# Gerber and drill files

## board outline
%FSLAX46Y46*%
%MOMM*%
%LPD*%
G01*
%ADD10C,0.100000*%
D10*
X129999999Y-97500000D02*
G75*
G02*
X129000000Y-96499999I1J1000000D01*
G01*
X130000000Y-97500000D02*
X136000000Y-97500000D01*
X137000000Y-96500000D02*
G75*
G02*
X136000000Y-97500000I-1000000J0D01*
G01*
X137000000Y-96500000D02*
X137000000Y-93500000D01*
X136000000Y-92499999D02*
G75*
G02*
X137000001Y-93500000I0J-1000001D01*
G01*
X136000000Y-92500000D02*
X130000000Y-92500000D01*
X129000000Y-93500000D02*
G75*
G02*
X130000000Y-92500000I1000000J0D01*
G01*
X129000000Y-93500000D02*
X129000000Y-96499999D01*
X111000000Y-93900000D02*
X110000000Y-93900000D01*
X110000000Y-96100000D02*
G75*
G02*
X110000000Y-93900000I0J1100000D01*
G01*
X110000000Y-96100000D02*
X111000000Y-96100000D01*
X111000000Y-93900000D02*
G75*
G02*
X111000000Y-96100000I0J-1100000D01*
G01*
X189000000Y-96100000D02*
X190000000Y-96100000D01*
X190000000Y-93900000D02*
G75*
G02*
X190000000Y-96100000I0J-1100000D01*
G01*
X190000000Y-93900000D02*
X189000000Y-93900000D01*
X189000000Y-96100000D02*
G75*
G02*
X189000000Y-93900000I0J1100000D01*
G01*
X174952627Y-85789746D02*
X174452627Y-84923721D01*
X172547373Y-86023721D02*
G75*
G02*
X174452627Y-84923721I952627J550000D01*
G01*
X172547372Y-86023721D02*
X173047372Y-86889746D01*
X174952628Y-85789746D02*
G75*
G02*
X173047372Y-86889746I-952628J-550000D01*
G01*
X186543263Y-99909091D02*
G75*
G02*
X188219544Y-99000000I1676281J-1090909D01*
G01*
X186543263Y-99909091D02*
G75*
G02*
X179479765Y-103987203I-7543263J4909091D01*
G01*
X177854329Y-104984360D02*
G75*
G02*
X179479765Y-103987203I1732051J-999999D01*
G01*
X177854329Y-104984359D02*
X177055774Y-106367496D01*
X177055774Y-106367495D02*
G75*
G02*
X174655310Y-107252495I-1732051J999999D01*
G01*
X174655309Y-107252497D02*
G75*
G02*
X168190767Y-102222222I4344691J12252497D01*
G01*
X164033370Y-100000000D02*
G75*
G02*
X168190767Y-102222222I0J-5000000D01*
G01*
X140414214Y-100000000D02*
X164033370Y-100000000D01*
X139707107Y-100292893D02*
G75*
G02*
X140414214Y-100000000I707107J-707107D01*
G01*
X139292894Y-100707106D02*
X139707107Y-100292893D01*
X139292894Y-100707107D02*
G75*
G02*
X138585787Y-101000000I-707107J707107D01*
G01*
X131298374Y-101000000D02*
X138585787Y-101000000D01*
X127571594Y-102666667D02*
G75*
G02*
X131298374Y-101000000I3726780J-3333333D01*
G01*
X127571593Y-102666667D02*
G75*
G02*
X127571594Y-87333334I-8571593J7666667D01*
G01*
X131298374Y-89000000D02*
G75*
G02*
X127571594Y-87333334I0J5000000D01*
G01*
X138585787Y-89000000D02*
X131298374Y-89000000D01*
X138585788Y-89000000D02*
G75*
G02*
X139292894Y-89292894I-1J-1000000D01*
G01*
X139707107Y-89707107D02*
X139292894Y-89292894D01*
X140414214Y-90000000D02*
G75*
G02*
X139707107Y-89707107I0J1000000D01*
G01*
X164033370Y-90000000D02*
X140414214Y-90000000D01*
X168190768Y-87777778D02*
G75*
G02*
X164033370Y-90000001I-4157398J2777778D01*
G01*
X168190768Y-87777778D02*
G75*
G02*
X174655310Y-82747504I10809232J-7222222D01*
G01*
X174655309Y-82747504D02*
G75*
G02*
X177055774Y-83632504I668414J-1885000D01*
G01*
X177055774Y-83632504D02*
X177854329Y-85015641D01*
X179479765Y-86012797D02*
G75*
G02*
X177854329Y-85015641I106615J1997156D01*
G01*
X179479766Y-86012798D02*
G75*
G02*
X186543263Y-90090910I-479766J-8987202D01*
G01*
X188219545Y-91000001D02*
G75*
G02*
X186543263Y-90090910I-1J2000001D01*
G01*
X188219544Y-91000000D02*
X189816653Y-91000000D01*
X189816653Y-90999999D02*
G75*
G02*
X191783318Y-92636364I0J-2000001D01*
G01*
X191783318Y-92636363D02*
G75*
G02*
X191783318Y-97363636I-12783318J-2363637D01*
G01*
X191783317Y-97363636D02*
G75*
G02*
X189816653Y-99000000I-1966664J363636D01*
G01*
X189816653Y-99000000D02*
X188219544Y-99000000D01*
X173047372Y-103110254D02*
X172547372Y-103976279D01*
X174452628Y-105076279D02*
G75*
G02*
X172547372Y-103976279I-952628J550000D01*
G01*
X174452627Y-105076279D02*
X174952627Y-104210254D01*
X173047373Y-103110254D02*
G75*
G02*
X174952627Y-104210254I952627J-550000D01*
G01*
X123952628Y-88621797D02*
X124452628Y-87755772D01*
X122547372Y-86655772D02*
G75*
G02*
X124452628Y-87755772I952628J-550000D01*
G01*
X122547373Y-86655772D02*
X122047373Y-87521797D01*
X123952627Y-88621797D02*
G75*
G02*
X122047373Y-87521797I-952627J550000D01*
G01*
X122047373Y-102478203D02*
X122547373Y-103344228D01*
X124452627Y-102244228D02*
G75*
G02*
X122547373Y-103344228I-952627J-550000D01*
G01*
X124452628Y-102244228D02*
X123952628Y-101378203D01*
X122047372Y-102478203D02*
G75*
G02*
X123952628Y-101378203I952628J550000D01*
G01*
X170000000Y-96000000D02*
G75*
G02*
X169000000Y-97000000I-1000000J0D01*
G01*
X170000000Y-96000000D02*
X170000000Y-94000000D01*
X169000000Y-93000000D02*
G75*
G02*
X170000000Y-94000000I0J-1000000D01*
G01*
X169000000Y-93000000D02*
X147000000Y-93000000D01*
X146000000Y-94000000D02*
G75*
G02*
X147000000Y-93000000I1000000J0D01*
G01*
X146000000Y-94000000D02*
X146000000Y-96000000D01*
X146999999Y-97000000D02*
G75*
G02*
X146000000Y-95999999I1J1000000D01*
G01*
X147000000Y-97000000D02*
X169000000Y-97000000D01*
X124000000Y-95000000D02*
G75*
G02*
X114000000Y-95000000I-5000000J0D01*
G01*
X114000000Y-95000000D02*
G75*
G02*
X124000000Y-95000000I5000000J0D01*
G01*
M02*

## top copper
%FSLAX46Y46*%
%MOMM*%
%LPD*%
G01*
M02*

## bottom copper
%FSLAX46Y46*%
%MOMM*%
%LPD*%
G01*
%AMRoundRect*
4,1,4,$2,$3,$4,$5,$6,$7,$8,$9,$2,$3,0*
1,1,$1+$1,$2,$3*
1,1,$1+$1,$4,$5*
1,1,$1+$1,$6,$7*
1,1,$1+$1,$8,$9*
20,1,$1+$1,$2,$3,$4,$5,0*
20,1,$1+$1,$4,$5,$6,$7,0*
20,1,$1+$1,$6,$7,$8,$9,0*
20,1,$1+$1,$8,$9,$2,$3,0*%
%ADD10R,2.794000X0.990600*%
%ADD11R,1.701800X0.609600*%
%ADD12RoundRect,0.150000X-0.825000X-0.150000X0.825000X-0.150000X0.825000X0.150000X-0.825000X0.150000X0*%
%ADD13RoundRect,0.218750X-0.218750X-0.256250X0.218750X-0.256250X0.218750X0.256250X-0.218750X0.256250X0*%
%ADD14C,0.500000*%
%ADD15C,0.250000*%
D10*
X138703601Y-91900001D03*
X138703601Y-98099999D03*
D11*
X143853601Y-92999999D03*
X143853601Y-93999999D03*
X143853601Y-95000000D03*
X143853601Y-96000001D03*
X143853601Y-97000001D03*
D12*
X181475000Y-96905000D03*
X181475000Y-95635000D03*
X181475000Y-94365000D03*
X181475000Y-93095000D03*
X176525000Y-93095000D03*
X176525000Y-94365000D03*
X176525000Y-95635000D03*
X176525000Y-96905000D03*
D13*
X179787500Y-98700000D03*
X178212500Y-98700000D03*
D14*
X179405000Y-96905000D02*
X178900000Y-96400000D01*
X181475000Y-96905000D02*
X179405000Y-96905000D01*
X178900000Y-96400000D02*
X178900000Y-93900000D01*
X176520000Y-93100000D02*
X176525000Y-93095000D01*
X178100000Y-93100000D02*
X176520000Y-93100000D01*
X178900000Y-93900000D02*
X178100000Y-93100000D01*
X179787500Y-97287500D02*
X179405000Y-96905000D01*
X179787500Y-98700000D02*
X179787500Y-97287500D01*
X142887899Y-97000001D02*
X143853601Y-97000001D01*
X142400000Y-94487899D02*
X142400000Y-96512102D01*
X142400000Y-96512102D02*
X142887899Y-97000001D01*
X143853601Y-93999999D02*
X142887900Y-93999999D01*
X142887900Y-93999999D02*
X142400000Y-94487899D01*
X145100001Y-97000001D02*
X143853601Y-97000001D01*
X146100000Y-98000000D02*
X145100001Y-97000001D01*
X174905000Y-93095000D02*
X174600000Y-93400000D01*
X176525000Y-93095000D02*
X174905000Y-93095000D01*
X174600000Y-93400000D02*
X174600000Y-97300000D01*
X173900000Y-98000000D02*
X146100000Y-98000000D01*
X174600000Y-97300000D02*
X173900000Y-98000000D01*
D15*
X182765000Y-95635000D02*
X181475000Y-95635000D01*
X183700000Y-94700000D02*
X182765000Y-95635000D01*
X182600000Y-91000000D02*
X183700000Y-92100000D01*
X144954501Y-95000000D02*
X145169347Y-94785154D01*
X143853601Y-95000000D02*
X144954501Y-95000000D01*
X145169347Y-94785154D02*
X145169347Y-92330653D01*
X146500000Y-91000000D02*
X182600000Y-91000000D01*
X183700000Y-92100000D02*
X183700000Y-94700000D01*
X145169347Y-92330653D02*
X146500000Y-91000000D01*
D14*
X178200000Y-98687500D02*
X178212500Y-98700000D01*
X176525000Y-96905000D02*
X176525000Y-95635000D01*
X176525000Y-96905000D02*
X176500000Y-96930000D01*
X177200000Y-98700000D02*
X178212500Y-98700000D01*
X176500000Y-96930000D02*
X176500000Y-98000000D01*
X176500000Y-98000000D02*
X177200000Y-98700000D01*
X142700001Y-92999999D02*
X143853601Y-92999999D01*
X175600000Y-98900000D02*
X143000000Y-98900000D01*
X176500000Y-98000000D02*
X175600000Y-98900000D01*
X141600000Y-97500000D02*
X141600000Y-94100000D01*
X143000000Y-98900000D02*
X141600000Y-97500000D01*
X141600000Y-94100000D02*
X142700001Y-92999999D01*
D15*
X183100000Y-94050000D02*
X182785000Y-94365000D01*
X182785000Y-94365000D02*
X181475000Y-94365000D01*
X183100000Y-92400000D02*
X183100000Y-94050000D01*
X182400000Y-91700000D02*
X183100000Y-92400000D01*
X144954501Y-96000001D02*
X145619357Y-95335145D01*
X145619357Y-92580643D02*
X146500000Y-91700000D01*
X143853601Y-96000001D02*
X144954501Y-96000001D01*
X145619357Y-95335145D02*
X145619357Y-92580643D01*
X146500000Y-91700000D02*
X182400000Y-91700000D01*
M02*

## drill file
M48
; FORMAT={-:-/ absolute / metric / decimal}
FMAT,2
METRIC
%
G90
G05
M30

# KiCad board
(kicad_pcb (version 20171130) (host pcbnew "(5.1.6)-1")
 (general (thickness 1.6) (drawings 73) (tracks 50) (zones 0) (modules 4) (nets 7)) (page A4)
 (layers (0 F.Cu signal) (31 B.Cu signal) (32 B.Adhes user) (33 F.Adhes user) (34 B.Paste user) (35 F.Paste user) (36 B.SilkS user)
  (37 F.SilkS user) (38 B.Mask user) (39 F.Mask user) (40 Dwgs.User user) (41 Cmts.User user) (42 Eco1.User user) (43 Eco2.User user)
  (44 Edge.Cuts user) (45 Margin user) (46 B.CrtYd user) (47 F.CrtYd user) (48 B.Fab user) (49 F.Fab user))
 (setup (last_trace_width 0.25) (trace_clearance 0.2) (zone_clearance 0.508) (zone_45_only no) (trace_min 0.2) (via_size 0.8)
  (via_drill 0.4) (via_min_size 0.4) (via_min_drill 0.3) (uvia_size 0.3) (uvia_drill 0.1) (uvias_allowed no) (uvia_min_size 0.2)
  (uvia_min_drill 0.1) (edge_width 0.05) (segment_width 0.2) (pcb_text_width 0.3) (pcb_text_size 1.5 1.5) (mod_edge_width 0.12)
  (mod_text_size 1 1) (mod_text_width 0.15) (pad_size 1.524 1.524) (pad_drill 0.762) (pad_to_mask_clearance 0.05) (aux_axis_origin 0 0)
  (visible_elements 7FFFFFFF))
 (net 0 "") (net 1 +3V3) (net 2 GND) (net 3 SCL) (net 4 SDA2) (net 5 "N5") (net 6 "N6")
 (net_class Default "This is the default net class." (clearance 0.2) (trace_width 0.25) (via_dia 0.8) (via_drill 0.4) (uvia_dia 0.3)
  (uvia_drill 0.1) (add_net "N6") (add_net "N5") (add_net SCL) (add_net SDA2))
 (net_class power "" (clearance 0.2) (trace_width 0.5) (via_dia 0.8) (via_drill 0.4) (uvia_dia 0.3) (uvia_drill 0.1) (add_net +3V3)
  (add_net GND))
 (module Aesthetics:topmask (layer F.Cu) (at 148.8 96.7)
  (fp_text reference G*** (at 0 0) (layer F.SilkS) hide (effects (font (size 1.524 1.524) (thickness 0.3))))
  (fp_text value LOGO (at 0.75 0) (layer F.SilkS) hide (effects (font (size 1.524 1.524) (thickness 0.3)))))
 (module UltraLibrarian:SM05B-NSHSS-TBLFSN (layer B.Cu) (at 141 95 90)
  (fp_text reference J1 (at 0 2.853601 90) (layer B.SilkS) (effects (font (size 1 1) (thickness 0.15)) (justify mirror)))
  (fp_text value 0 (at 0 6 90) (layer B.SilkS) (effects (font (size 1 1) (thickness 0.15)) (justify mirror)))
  (pad 7 smd rect (at 3.099999 -2.296399 90) (size 0.9906 2.794) (layers B.Cu B.Paste B.Mask))
  (pad 6 smd rect (at -3.099999 -2.296399 90) (size 0.9906 2.794) (layers B.Cu B.Paste B.Mask))
  (pad 5 smd rect (at 2.000001 2.853601 90) (size 0.6096 1.7018) (layers B.Cu B.Paste B.Mask) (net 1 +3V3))
  (pad 4 smd rect (at 1.000001 2.853601 90) (size 0.6096 1.7018) (layers B.Cu B.Paste B.Mask) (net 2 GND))
  (pad 3 smd rect (at 0 2.853601 90) (size 0.6096 1.7018) (layers B.Cu B.Paste B.Mask) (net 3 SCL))
  (pad 2 smd rect (at -1.000001 2.853601 90) (size 0.6096 1.7018) (layers B.Cu B.Paste B.Mask) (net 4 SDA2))
  (pad 1 smd rect (at -2.000001 2.853601 90) (size 0.6096 1.7018) (layers B.Cu B.Paste B.Mask) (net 2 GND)))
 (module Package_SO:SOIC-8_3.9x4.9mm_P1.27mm (layer B.Cu) (at 179 95)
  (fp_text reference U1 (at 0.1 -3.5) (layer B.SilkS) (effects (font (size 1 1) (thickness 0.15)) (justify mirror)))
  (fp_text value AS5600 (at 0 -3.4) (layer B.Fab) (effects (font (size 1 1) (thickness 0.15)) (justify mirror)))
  (pad 8 smd roundrect (at 2.475 1.905) (size 1.95 0.6) (layers B.Cu B.Paste B.Mask) (roundrect_rratio 0.25) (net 2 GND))
  (pad 7 smd roundrect (at 2.475 0.635) (size 1.95 0.6) (layers B.Cu B.Paste B.Mask) (roundrect_rratio 0.25) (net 3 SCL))
  (pad 6 smd roundrect (at 2.475 -0.635) (size 1.95 0.6) (layers B.Cu B.Paste B.Mask) (roundrect_rratio 0.25) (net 4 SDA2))
  (pad 5 smd roundrect (at 2.475 -1.905) (size 1.95 0.6) (layers B.Cu B.Paste B.Mask) (roundrect_rratio 0.25) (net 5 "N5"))
  (pad 4 smd roundrect (at -2.475 -1.905) (size 1.95 0.6) (layers B.Cu B.Paste B.Mask) (roundrect_rratio 0.25) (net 2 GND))
  (pad 3 smd roundrect (at -2.475 -0.635) (size 1.95 0.6) (layers B.Cu B.Paste B.Mask) (roundrect_rratio 0.25) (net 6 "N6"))
  (pad 2 smd roundrect (at -2.475 0.635) (size 1.95 0.6) (layers B.Cu B.Paste B.Mask) (roundrect_rratio 0.25) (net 1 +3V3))
  (pad 1 smd roundrect (at -2.475 1.905) (size 1.95 0.6) (layers B.Cu B.Paste B.Mask) (roundrect_rratio 0.25) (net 1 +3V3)))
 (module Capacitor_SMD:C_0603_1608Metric (layer B.Cu) (at 179 98.7)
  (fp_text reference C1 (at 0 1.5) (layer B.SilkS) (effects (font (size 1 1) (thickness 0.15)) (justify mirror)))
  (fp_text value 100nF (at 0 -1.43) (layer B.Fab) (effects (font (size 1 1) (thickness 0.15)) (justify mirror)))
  (pad 2 smd roundrect (at 0.7875 0) (size 0.875 0.95) (layers B.Cu B.Paste B.Mask) (roundrect_rratio 0.25) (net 2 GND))
  (pad 1 smd roundrect (at -0.7875 0) (size 0.875 0.95) (layers B.Cu B.Paste B.Mask) (roundrect_rratio 0.25) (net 1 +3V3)))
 (gr_arc (start 130 96.5) (end 129 96.499999) (angle -90) (layer Edge.Cuts) (width 0.1))
 (gr_line (start 130 97.5) (end 136 97.5) (layer Edge.Cuts) (width 0.1))
 (gr_arc (start 136 96.5) (end 136 97.5) (angle -90) (layer Edge.Cuts) (width 0.1))
 (gr_line (start 137 96.5) (end 137 93.5) (layer Edge.Cuts) (width 0.1))
 (gr_arc (start 136 93.5) (end 137.000001 93.5) (angle -90) (layer Edge.Cuts) (width 0.1))
 (gr_line (start 136 92.5) (end 130 92.5) (layer Edge.Cuts) (width 0.1))
 (gr_arc (start 130 93.5) (end 130 92.5) (angle -90) (layer Edge.Cuts) (width 0.1))
 (gr_line (start 129 93.5) (end 129 96.499999) (layer Edge.Cuts) (width 0.1))
 (gr_line (start 111 93.9) (end 110 93.9) (layer Edge.Cuts) (width 0.1))
 (gr_arc (start 110 95) (end 110 93.9) (angle -180) (layer Edge.Cuts) (width 0.1))
 (gr_line (start 110 96.1) (end 111 96.1) (layer Edge.Cuts) (width 0.1))
 (gr_arc (start 111 95) (end 111 96.1) (angle -180) (layer Edge.Cuts) (width 0.1))
 (gr_line (start 189 96.1) (end 190 96.1) (layer Edge.Cuts) (width 0.1))
 (gr_arc (start 190 95) (end 190 96.1) (angle -180) (layer Edge.Cuts) (width 0.1))
 (gr_line (start 190 93.9) (end 189 93.9) (layer Edge.Cuts) (width 0.1))
 (gr_arc (start 189 95) (end 189 93.9) (angle -180) (layer Edge.Cuts) (width 0.1))
 (gr_line (start 174.952627 85.789746) (end 174.452627 84.923721) (layer Edge.Cuts) (width 0.1))
 (gr_arc (start 173.5 85.473721) (end 174.452627 84.923721) (angle -180) (layer Edge.Cuts) (width 0.1))
 (gr_line (start 172.547372 86.023721) (end 173.047372 86.889746) (layer Edge.Cuts) (width 0.1))
 (gr_arc (start 174 86.339746) (end 173.047372 86.889746) (angle -180) (layer Edge.Cuts) (width 0.1))
 (gr_arc (start 188.219544 101) (end 188.219544 99) (angle -56.94426885) (layer Edge.Cuts) (width 0.1))
 (gr_arc (start 179 95) (end 179.479765 103.987203) (angle -53.8885377) (layer Edge.Cuts) (width 0.1))
 (gr_arc (start 179.58638 105.984359) (end 179.479765 103.987203) (angle -56.94426885) (layer Edge.Cuts) (width 0.1))
 (gr_line (start 177.854329 104.984359) (end 177.055774 106.367496) (layer Edge.Cuts) (width 0.1))
 (gr_arc (start 175.323723 105.367496) (end 174.65531 107.252496) (angle -79.5243183) (layer Edge.Cuts) (width 0.1))
 (gr_arc (start 179 95) (end 168.190767 102.222222) (angle -36.7266931) (layer Edge.Cuts) (width 0.1))
 (gr_arc (start 164.03337 105) (end 168.190767 102.222222) (angle -56.2510114) (layer Edge.Cuts) (width 0.1))
 (gr_line (start 140.414214 100) (end 164.03337 100) (layer Edge.Cuts) (width 0.1))
 (gr_arc (start 140.414214 101) (end 140.414214 99.999999) (angle -45) (layer Edge.Cuts) (width 0.1))
 (gr_line (start 139.292894 100.707106) (end 139.707107 100.292893) (layer Edge.Cuts) (width 0.1))
 (gr_arc (start 138.585787 100) (end 138.585787 101) (angle -45) (layer Edge.Cuts) (width 0.1))
 (gr_line (start 131.298374 101) (end 138.585787 101) (layer Edge.Cuts) (width 0.1))
 (gr_arc (start 131.298374 106) (end 131.298374 101) (angle -48.1896851) (layer Edge.Cuts) (width 0.1))
 (gr_arc (start 119 95) (end 127.571594 87.333334) (angle -276.3793702) (layer Edge.Cuts) (width 0.1))
 (gr_arc (start 131.298374 84) (end 127.571594 87.333334) (angle -48.1896851) (layer Edge.Cuts) (width 0.1))
 (gr_line (start 138.585787 89) (end 131.298374 89) (layer Edge.Cuts) (width 0.1))
 (gr_arc (start 138.585787 90) (end 139.292894 89.292894) (angle -45) (layer Edge.Cuts) (width 0.1))
 (gr_line (start 139.707107 89.707107) (end 139.292894 89.292894) (layer Edge.Cuts) (width 0.1))
 (gr_arc (start 140.414214 89) (end 139.707107 89.707107) (angle -45) (layer Edge.Cuts) (width 0.1))
 (gr_line (start 164.03337 90) (end 140.414214 90) (layer Edge.Cuts) (width 0.1))
 (gr_arc (start 164.03337 85) (end 164.03337 90.000001) (angle -56.2510114) (layer Edge.Cuts) (width 0.1))
 (gr_arc (start 179 95) (end 174.65531 82.747504) (angle -36.7266931) (layer Edge.Cuts) (width 0.1))
 (gr_arc (start 175.323723 84.632504) (end 177.055774 83.632504) (angle -79.5243183) (layer Edge.Cuts) (width 0.1))
 (gr_line (start 177.055774 83.632504) (end 177.854329 85.015641) (layer Edge.Cuts) (width 0.1))
 (gr_arc (start 179.58638 84.015641) (end 177.854329 85.015641) (angle -56.94426885) (layer Edge.Cuts) (width 0.1))
 (gr_arc (start 179 95) (end 186.543263 90.09091) (angle -53.8885377) (layer Edge.Cuts) (width 0.1))
 (gr_arc (start 188.219544 89) (end 186.543263 90.09091) (angle -56.94426885) (layer Edge.Cuts) (width 0.1))
 (gr_line (start 188.219544 91) (end 189.816653 91) (layer Edge.Cuts) (width 0.1))
 (gr_arc (start 189.816653 93) (end 191.783318 92.636364) (angle -79.5243183) (layer Edge.Cuts) (width 0.1))
 (gr_arc (start 179 95) (end 191.783318 97.363636) (angle -20.95136339) (layer Edge.Cuts) (width 0.1))
 (gr_arc (start 189.816653 97) (end 189.816653 99) (angle -79.5243183) (layer Edge.Cuts) (width 0.1))
 (gr_line (start 189.816653 99) (end 188.219544 99) (layer Edge.Cuts) (width 0.1))
 (gr_line (start 173.047372 103.110254) (end 172.547372 103.976279) (layer Edge.Cuts) (width 0.1))
 (gr_arc (start 173.5 104.526279) (end 172.547372 103.976279) (angle -180) (layer Edge.Cuts) (width 0.1))
 (gr_line (start 174.452627 105.076279) (end 174.952627 104.210254) (layer Edge.Cuts) (width 0.1))
 (gr_arc (start 174 103.660254) (end 174.952627 104.210254) (angle -180) (layer Edge.Cuts) (width 0.1))
 (gr_line (start 123.952628 88.621797) (end 124.452628 87.755772) (layer Edge.Cuts) (width 0.1))
 (gr_arc (start 123.5 87.205772) (end 124.452628 87.755772) (angle -180) (layer Edge.Cuts) (width 0.1))
 (gr_line (start 122.547373 86.655772) (end 122.047373 87.521797) (layer Edge.Cuts) (width 0.1))
 (gr_arc (start 123 88.071797) (end 122.047373 87.521797) (angle -180) (layer Edge.Cuts) (width 0.1))
 (gr_line (start 122.047373 102.478203) (end 122.547373 103.344228) (layer Edge.Cuts) (width 0.1))
 (gr_arc (start 123.5 102.794228) (end 122.547373 103.344228) (angle -180) (layer Edge.Cuts) (width 0.1))
 (gr_line (start 124.452628 102.244228) (end 123.952628 101.378203) (layer Edge.Cuts) (width 0.1))
 (gr_arc (start 123 101.928203) (end 123.952628 101.378203) (angle -180) (layer Edge.Cuts) (width 0.1))
 (gr_arc (start 169 96) (end 169 97) (angle -90) (layer Edge.Cuts) (width 0.1))
 (gr_line (start 170 96) (end 170 94) (layer Edge.Cuts) (width 0.1))
 (gr_arc (start 169 94) (end 170 94) (angle -90) (layer Edge.Cuts) (width 0.1))
 (gr_line (start 169 93) (end 147 93) (layer Edge.Cuts) (width 0.1))
 (gr_arc (start 147 94) (end 147 93) (angle -90) (layer Edge.Cuts) (width 0.1))
 (gr_line (start 146 94) (end 146 96) (layer Edge.Cuts) (width 0.1))
 (gr_arc (start 147 96) (end 146 95.999999) (angle -90) (layer Edge.Cuts) (width 0.1))
 (gr_line (start 147 97) (end 169 97) (layer Edge.Cuts) (width 0.1))
 (gr_circle (center 119 95) (end 124 95) (layer Edge.Cuts) (width 0.1))
 (segment (start 179.405 96.905) (end 178.9 96.4) (width 0.5) (layer B.Cu) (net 2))
 (segment (start 181.475 96.905) (end 179.405 96.905) (width 0.5) (layer B.Cu) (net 2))
 (segment (start 178.9 96.4) (end 178.9 93.9) (width 0.5) (layer B.Cu) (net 2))
 (segment (start 176.52 93.1) (end 176.525 93.095) (width 0.5) (layer B.Cu) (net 2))
 (segment (start 178.1 93.1) (end 176.52 93.1) (width 0.5) (layer B.Cu) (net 2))
 (segment (start 178.9 93.9) (end 178.1 93.1) (width 0.5) (layer B.Cu) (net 2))
 (segment (start 179.7875 97.2875) (end 179.405 96.905) (width 0.5) (layer B.Cu) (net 2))
 (segment (start 179.7875 98.7) (end 179.7875 97.2875) (width 0.5) (layer B.Cu) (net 2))
 (segment (start 142.887899 97.000001) (end 143.853601 97.000001) (width 0.5) (layer B.Cu) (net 2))
 (segment (start 142.4 94.487899) (end 142.4 96.512102) (width 0.5) (layer B.Cu) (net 2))
 (segment (start 142.4 96.512102) (end 142.887899 97.000001) (width 0.5) (layer B.Cu) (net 2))
 (segment (start 143.853601 93.999999) (end 142.8879 93.999999) (width 0.5) (layer B.Cu) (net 2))
 (segment (start 142.8879 93.999999) (end 142.4 94.487899) (width 0.5) (layer B.Cu) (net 2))
 (segment (start 145.100001 97.000001) (end 143.853601 97.000001) (width 0.5) (layer B.Cu) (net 2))
 (segment (start 146.1 98) (end 145.100001 97.000001) (width 0.5) (layer B.Cu) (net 2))
 (segment (start 174.905 93.095) (end 174.6 93.4) (width 0.5) (layer B.Cu) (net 2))
 (segment (start 176.525 93.095) (end 174.905 93.095) (width 0.5) (layer B.Cu) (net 2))
 (segment (start 174.6 93.4) (end 174.6 97.3) (width 0.5) (layer B.Cu) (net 2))
 (segment (start 173.9 98) (end 146.1 98) (width 0.5) (layer B.Cu) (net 2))
 (segment (start 174.6 97.3) (end 173.9 98) (width 0.5) (layer B.Cu) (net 2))
 (segment (start 182.765 95.635) (end 181.475 95.635) (width 0.25) (layer B.Cu) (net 3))
 (segment (start 183.7 94.7) (end 182.765 95.635) (width 0.25) (layer B.Cu) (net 3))
 (segment (start 182.6 91) (end 183.7 92.1) (width 0.25) (layer B.Cu) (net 3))
 (segment (start 144.954501 95) (end 145.169347 94.785154) (width 0.25) (layer B.Cu) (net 3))
 (segment (start 143.853601 95) (end 144.954501 95) (width 0.25) (layer B.Cu) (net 3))
 (segment (start 145.169347 94.785154) (end 145.169347 92.330653) (width 0.25) (layer B.Cu) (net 3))
 (segment (start 146.5 91) (end 182.6 91) (width 0.25) (layer B.Cu) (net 3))
 (segment (start 183.7 92.1) (end 183.7 94.7) (width 0.25) (layer B.Cu) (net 3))
 (segment (start 145.169347 92.330653) (end 146.5 91) (width 0.25) (layer B.Cu) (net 3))
 (segment (start 178.2 98.6875) (end 178.2125 98.7) (width 0.5) (layer B.Cu) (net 1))
 (segment (start 176.525 96.905) (end 176.525 95.635) (width 0.5) (layer B.Cu) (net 1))
 (segment (start 176.525 96.905) (end 176.5 96.93) (width 0.5) (layer B.Cu) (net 1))
 (segment (start 177.2 98.7) (end 178.2125 98.7) (width 0.5) (layer B.Cu) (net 1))
 (segment (start 176.5 96.93) (end 176.5 98) (width 0.5) (layer B.Cu) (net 1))
 (segment (start 176.5 98) (end 177.2 98.7) (width 0.5) (layer B.Cu) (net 1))
 (segment (start 142.700001 92.999999) (end 143.853601 92.999999) (width 0.5) (layer B.Cu) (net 1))
 (segment (start 175.6 98.9) (end 143 98.9) (width 0.5) (layer B.Cu) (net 1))
 (segment (start 176.5 98) (end 175.6 98.9) (width 0.5) (layer B.Cu) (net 1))
 (segment (start 141.6 97.5) (end 141.6 94.1) (width 0.5) (layer B.Cu) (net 1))
 (segment (start 143 98.9) (end 141.6 97.5) (width 0.5) (layer B.Cu) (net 1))
 (segment (start 141.6 94.1) (end 142.700001 92.999999) (width 0.5) (layer B.Cu) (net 1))
 (segment (start 183.1 94.05) (end 182.785 94.365) (width 0.25) (layer B.Cu) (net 4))
 (segment (start 182.785 94.365) (end 181.475 94.365) (width 0.25) (layer B.Cu) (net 4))
 (segment (start 183.1 92.4) (end 183.1 94.05) (width 0.25) (layer B.Cu) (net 4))
 (segment (start 182.4 91.7) (end 183.1 92.4) (width 0.25) (layer B.Cu) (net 4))
 (segment (start 144.954501 96.000001) (end 145.619357 95.335145) (width 0.25) (layer B.Cu) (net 4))
 (segment (start 145.619357 92.580643) (end 146.5 91.7) (width 0.25) (layer B.Cu) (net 4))
 (segment (start 143.853601 96.000001) (end 144.954501 96.000001) (width 0.25) (layer B.Cu) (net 4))
 (segment (start 145.619357 95.335145) (end 145.619357 92.580643) (width 0.25) (layer B.Cu) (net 4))
 (segment (start 146.5 91.7) (end 182.4 91.7) (width 0.25) (layer B.Cu) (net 4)))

